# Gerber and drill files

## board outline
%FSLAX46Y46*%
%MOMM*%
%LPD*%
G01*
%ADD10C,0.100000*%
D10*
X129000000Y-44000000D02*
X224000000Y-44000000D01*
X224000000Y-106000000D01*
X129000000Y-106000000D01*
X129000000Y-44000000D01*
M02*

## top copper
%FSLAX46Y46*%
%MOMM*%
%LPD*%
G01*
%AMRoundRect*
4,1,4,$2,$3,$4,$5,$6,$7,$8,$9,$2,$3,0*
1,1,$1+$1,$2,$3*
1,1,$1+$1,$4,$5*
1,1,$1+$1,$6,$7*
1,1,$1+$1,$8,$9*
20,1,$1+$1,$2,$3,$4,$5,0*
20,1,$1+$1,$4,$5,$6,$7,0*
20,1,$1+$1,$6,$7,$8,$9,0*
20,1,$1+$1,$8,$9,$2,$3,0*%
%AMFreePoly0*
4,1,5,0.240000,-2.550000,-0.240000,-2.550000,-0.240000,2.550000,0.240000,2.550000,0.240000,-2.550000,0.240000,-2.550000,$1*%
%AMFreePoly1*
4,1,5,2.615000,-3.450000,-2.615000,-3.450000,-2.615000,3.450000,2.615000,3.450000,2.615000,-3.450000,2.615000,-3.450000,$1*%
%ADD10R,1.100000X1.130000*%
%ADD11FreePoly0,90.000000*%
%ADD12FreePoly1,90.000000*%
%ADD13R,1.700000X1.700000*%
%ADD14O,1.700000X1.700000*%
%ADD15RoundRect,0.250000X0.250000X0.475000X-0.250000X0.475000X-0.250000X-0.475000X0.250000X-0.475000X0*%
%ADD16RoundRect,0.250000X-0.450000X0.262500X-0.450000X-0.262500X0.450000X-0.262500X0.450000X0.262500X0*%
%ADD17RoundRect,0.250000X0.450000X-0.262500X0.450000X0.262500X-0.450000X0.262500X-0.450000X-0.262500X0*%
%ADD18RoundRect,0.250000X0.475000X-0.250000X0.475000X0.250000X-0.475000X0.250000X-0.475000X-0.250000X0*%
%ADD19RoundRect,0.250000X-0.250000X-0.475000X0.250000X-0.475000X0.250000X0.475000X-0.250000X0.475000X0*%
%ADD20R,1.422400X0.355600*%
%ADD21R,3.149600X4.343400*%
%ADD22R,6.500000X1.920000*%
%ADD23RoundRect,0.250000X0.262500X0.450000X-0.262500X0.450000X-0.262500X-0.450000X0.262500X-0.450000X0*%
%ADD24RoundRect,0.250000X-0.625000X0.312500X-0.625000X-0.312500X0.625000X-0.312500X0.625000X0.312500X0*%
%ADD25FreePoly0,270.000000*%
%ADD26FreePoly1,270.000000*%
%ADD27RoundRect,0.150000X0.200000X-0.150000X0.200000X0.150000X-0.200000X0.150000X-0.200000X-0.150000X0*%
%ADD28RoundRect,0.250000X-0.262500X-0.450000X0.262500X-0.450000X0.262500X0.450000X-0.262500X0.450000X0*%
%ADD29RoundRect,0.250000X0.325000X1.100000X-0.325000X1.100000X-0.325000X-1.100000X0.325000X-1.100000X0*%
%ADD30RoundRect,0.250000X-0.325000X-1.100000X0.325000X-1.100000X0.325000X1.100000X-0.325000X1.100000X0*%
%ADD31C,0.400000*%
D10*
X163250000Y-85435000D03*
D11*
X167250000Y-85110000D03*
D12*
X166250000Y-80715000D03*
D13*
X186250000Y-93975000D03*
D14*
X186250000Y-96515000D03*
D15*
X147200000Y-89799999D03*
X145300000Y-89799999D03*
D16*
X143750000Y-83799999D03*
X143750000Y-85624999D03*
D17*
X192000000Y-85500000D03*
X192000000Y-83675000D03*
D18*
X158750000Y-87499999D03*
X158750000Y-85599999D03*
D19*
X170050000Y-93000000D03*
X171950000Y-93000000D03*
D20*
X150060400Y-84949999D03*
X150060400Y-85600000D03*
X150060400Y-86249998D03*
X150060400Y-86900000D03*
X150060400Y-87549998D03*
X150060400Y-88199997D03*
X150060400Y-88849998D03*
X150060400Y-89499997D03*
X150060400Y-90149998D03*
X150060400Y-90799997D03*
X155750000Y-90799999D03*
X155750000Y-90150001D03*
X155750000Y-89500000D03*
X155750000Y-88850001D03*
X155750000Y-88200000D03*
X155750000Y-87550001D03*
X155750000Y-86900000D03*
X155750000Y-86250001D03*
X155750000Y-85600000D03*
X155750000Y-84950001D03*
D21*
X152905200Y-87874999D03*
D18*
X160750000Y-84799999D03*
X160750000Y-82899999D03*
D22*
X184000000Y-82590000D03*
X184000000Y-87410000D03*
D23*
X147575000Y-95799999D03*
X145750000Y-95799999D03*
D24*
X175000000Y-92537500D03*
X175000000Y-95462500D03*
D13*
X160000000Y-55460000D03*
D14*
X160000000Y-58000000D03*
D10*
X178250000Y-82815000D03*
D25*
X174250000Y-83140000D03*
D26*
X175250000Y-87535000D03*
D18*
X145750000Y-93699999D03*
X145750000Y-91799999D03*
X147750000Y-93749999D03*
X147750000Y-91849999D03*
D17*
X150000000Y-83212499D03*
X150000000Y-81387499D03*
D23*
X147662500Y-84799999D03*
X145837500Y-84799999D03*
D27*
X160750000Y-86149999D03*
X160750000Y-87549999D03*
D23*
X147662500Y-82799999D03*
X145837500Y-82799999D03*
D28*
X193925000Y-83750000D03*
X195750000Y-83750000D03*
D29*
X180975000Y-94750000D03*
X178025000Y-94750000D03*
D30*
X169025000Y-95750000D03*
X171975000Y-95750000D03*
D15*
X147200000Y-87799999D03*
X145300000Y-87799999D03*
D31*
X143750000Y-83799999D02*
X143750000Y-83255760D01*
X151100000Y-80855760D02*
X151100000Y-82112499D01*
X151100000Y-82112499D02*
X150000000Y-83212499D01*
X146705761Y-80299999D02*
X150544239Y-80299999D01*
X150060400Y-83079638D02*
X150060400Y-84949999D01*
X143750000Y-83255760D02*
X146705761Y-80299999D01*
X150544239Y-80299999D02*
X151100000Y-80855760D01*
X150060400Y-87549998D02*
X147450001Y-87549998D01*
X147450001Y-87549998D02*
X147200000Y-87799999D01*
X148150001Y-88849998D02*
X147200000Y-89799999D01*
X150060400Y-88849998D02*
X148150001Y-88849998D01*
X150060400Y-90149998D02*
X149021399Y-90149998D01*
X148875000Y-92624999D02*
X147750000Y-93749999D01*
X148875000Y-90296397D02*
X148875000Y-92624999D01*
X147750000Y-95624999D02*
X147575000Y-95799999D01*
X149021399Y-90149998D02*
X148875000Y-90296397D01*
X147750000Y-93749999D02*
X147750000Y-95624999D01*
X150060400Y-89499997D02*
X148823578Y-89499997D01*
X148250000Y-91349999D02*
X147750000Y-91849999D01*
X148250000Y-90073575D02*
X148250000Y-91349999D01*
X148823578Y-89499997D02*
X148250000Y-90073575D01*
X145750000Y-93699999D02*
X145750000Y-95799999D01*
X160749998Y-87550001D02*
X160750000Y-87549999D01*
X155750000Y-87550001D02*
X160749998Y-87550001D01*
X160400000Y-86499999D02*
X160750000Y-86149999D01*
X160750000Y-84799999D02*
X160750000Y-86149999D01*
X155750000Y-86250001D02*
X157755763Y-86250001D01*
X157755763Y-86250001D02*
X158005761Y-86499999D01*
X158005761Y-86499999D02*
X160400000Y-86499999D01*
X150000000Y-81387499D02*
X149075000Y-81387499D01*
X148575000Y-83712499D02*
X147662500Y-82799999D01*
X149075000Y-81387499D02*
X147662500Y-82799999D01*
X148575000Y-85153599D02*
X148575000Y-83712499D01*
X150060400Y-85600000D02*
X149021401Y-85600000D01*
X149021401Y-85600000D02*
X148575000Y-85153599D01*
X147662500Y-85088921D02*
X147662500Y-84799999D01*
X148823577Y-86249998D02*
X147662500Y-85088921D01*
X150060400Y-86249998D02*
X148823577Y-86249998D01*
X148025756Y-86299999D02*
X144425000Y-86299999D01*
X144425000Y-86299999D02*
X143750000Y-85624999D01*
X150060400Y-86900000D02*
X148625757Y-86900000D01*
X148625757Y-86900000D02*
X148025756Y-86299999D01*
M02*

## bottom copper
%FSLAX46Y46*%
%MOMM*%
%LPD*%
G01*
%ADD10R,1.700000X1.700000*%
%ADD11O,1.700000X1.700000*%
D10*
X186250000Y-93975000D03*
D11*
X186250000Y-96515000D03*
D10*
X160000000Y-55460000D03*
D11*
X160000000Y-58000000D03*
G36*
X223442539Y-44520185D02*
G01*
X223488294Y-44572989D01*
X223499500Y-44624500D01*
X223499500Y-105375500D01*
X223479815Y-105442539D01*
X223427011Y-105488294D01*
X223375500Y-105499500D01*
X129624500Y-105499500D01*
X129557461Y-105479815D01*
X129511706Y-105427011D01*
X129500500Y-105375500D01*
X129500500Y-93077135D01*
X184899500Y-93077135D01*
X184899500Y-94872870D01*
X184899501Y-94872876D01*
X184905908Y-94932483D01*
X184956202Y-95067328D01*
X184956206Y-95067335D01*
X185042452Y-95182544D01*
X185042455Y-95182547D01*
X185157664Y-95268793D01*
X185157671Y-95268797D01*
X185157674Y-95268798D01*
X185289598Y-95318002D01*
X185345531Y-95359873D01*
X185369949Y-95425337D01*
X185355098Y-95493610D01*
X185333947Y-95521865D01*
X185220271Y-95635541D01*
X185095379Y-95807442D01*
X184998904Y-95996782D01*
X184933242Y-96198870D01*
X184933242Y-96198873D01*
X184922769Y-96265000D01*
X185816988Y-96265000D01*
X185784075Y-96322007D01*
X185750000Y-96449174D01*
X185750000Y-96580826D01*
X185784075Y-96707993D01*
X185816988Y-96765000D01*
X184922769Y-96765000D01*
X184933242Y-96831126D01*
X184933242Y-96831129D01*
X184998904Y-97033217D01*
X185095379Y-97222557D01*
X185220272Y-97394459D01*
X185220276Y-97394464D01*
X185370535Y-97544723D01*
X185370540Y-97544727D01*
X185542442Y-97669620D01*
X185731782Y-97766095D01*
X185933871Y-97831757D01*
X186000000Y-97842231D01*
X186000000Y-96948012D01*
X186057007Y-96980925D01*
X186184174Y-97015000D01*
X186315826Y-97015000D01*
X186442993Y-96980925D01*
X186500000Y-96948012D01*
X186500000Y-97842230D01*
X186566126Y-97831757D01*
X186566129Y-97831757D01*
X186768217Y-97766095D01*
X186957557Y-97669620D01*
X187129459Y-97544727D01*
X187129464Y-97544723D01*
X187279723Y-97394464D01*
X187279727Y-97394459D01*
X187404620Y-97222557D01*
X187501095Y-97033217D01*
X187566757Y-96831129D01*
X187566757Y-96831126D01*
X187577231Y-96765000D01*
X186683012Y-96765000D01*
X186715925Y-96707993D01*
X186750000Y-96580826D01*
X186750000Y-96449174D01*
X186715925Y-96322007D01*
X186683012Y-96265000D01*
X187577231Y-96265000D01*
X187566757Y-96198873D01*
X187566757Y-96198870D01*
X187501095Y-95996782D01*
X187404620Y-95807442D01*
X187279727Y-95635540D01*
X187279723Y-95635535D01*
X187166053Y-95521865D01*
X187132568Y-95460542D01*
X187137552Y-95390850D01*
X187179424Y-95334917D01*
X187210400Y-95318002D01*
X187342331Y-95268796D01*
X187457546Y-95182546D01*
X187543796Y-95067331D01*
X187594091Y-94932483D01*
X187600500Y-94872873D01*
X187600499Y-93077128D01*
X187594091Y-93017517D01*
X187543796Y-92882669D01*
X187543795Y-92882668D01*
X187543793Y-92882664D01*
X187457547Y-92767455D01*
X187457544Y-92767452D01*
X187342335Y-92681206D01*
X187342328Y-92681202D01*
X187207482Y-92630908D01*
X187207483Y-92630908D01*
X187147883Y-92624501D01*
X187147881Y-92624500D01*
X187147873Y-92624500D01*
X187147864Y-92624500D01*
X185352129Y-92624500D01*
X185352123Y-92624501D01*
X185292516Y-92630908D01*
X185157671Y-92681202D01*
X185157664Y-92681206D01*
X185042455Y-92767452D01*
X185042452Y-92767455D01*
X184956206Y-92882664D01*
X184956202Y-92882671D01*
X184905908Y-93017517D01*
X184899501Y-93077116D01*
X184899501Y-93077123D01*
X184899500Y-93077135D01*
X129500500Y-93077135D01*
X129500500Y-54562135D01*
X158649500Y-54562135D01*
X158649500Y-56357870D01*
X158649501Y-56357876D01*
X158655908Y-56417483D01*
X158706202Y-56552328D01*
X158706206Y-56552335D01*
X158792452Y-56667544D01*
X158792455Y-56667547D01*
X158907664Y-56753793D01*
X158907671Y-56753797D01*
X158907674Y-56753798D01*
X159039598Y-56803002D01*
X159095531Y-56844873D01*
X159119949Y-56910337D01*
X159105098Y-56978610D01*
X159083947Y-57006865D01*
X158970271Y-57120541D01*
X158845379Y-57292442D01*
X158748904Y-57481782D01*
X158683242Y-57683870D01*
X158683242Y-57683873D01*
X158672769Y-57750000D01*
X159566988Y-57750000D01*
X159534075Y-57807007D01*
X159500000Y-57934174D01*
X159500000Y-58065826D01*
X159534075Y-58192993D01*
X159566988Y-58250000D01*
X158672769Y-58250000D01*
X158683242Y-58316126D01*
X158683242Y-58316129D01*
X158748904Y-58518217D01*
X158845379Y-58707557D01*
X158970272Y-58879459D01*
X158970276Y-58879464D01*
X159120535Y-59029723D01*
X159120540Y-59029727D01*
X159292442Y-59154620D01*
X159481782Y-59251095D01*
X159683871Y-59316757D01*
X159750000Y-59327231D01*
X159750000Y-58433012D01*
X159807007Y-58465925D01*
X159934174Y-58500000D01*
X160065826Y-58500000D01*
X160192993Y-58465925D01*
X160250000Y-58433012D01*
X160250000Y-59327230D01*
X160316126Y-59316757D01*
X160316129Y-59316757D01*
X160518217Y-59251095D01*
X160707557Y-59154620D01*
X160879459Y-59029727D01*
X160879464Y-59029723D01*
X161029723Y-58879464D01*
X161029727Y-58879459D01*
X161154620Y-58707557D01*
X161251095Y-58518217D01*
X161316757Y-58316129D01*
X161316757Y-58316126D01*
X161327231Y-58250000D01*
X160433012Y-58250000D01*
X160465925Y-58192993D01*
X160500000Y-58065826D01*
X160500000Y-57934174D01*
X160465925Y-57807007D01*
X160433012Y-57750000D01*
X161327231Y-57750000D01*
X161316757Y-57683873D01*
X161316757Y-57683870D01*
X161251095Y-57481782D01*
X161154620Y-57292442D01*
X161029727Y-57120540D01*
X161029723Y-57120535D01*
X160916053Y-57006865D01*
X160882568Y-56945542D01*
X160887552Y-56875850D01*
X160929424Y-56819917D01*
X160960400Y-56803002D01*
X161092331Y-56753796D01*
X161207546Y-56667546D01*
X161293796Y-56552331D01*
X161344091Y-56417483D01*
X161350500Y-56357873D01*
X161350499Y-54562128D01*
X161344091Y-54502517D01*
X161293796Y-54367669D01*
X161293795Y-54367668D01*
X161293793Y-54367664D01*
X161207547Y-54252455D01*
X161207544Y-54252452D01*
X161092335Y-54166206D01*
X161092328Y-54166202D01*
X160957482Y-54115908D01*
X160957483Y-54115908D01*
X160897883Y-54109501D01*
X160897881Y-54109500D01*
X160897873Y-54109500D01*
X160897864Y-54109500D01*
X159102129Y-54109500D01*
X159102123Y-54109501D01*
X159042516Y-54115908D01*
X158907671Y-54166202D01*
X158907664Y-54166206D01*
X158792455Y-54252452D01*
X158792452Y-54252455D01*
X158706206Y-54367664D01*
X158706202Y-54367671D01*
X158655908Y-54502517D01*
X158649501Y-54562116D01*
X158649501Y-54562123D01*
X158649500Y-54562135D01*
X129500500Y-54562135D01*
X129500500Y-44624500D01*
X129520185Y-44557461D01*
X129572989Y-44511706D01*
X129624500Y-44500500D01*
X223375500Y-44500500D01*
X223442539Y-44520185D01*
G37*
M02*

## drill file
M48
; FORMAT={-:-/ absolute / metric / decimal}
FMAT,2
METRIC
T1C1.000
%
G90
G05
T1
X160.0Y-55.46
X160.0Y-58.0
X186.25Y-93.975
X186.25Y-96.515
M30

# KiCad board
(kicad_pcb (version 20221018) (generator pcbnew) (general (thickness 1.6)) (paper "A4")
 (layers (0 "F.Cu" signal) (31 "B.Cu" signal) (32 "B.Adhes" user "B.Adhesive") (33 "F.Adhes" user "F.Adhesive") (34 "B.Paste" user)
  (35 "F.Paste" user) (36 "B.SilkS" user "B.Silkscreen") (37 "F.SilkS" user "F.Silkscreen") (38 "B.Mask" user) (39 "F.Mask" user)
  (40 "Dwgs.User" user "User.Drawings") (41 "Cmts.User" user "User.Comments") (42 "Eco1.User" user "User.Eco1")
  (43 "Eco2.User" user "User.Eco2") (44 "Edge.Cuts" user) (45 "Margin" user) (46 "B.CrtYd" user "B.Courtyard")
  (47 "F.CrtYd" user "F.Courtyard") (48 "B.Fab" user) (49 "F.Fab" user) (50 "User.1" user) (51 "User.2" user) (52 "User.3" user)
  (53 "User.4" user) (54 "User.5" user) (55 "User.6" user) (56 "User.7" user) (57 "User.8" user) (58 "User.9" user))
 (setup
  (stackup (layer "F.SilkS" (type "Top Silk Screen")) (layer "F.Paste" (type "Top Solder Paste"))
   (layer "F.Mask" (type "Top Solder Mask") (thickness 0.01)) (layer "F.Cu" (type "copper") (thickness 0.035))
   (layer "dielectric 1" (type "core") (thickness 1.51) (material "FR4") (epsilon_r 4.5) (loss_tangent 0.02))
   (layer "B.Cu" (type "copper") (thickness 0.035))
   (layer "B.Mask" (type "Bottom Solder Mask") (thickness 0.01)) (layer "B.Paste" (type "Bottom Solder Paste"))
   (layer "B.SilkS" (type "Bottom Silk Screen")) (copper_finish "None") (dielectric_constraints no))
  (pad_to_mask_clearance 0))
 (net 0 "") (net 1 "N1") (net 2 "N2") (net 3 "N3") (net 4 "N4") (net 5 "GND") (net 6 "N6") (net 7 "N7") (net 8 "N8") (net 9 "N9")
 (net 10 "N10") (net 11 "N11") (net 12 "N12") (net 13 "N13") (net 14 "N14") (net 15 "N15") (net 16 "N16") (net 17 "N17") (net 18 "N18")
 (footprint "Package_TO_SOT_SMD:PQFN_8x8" (layer "F.Cu") (at 166.25 81.5 90)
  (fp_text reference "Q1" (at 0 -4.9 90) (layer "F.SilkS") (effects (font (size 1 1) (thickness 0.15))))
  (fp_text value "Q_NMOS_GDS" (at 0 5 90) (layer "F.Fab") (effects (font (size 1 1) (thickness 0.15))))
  (pad "" smd rect (at -0.5 -2.25) (size 1.5 1.5) (layers "F.Paste"))
  (pad "" smd rect (at -0.5 0) (size 1.5 1.5) (layers "F.Paste"))
  (pad "" smd rect (at -0.5 2.25) (size 1.5 1.5) (layers "F.Paste"))
  (pad "" smd rect (at 2 -2.25) (size 1.5 1.5) (layers "F.Paste")) (pad "" smd rect (at 2 0) (size 1.5 1.5) (layers "F.Paste"))
  (pad "" smd rect (at 2 2.25) (size 1.5 1.5) (layers "F.Paste"))
  (pad "1" smd rect (at -3.935 -3 90) (size 1.13 1.1) (layers "F.Cu" "F.Paste" "F.Mask") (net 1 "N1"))
  (pad "2" smd custom (at -3.61 1 90) (size 0.48 5.1) (layers "F.Cu" "F.Paste" "F.Mask") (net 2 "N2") (zone_connect 2)
   (thermal_bridge_angle 45) (options (clearance outline) (anchor rect)) (primitives))
  (pad "3" smd custom (at 0.785 0 90) (size 5.23 6.9) (layers "F.Cu" "F.Mask") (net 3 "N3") (zone_connect 2) (thermal_bridge_angle 45)
   (options (clearance outline) (anchor rect)) (primitives)))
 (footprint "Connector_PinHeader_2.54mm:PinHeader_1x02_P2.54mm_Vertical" (layer "F.Cu") (at 186.25 93.975)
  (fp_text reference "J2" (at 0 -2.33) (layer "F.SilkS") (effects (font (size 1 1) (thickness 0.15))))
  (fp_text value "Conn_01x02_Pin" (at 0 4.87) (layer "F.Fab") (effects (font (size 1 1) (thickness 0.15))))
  (pad "1" thru_hole rect (at 0 0) (size 1.7 1.7) (drill 1) (layers "*.Cu" "*.Mask") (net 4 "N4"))
  (pad "2" thru_hole oval (at 0 2.54) (size 1.7 1.7) (drill 1) (layers "*.Cu" "*.Mask") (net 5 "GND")))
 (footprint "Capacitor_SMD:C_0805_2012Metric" (layer "F.Cu") (at 146.25 89.799999 180)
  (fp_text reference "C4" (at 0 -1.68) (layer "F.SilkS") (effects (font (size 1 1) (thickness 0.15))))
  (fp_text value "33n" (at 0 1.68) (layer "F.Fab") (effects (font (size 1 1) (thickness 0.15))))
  (pad "1" smd roundrect (at -0.95 0 180) (size 1 1.45) (layers "F.Cu" "F.Paste" "F.Mask") (roundrect_rratio 0.25) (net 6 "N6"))
  (pad "2" smd roundrect (at 0.95 0 180) (size 1 1.45) (layers "F.Cu" "F.Paste" "F.Mask") (roundrect_rratio 0.25) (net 5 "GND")))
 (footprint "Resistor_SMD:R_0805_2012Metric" (layer "F.Cu") (at 143.75 84.712499 -90)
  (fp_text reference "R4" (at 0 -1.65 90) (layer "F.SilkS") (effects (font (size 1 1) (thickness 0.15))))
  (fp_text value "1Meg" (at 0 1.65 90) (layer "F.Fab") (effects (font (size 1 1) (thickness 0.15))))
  (pad "1" smd roundrect (at -0.9125 0 270) (size 1.025 1.4) (layers "F.Cu" "F.Paste" "F.Mask") (roundrect_rratio 0.243902) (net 2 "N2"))
  (pad "2" smd roundrect (at 0.9125 0 270) (size 1.025 1.4) (layers "F.Cu" "F.Paste" "F.Mask") (roundrect_rratio 0.243902) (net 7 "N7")))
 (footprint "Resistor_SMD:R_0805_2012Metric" (layer "F.Cu") (at 192 84.5875 90)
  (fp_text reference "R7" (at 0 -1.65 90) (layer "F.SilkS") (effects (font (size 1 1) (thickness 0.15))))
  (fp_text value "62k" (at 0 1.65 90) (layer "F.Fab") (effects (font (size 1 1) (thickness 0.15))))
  (pad "1" smd roundrect (at -0.9125 0 90) (size 1.025 1.4) (layers "F.Cu" "F.Paste" "F.Mask") (roundrect_rratio 0.243902) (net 4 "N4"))
  (pad "2" smd roundrect (at 0.9125 0 90) (size 1.025 1.4) (layers "F.Cu" "F.Paste" "F.Mask") (roundrect_rratio 0.243902) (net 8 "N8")))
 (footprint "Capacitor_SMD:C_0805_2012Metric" (layer "F.Cu") (at 158.75 86.549999 90)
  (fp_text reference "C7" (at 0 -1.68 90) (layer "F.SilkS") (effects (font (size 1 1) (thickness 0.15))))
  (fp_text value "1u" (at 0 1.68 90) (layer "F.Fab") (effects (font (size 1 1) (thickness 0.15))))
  (pad "1" smd roundrect (at -0.95 0 90) (size 1 1.45) (layers "F.Cu" "F.Paste" "F.Mask") (roundrect_rratio 0.25) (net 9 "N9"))
  (pad "2" smd roundrect (at 0.95 0 90) (size 1 1.45) (layers "F.Cu" "F.Paste" "F.Mask") (roundrect_rratio 0.25) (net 5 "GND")))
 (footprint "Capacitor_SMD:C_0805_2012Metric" (layer "F.Cu") (at 171 93)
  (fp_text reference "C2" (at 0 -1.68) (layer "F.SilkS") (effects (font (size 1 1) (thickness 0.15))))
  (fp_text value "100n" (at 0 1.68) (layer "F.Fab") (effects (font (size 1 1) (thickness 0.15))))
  (pad "1" smd roundrect (at -0.95 0) (size 1 1.45) (layers "F.Cu" "F.Paste" "F.Mask") (roundrect_rratio 0.25) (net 2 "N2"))
  (pad "2" smd roundrect (at 0.95 0) (size 1 1.45) (layers "F.Cu" "F.Paste" "F.Mask") (roundrect_rratio 0.25) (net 5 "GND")))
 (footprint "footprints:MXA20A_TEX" (layer "F.Cu") (at 152.9052 87.874999)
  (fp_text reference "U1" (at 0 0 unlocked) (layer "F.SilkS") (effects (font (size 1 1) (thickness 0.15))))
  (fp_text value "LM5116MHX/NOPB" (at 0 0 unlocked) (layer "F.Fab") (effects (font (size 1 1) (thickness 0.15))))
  (pad "1" smd rect (at -2.8448 -2.925) (size 1.4224 0.3556) (layers "F.Cu" "F.Paste" "F.Mask") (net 2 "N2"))
  (pad "2" smd rect (at -2.8448 -2.274999) (size 1.4224 0.3556) (layers "F.Cu" "F.Paste" "F.Mask") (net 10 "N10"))
  (pad "3" smd rect (at -2.8448 -1.625001) (size 1.4224 0.3556) (layers "F.Cu" "F.Paste" "F.Mask") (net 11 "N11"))
  (pad "4" smd rect (at -2.8448 -0.974999) (size 1.4224 0.3556) (layers "F.Cu" "F.Paste" "F.Mask") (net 7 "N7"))
  (pad "5" smd rect (at -2.8448 -0.325001) (size 1.4224 0.3556) (layers "F.Cu" "F.Paste" "F.Mask") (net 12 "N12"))
  (pad "6" smd rect (at -2.8448 0.324998) (size 1.4224 0.3556) (layers "F.Cu" "F.Paste" "F.Mask") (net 5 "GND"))
  (pad "7" smd rect (at -2.8448 0.974999) (size 1.4224 0.3556) (layers "F.Cu" "F.Paste" "F.Mask") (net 6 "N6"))
  (pad "8" smd rect (at -2.8448 1.624998) (size 1.4224 0.3556) (layers "F.Cu" "F.Paste" "F.Mask") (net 8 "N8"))
  (pad "9" smd rect (at -2.8448 2.274999) (size 1.4224 0.3556) (layers "F.Cu" "F.Paste" "F.Mask") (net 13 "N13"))
  (pad "10" smd rect (at -2.8448 2.924998) (size 1.4224 0.3556) (layers "F.Cu" "F.Paste" "F.Mask") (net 4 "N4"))
  (pad "11" smd rect (at 2.8448 2.925) (size 1.4224 0.3556) (layers "F.Cu" "F.Paste" "F.Mask") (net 5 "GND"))
  (pad "12" smd rect (at 2.8448 2.275002) (size 1.4224 0.3556) (layers "F.Cu" "F.Paste" "F.Mask") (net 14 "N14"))
  (pad "13" smd rect (at 2.8448 1.625001) (size 1.4224 0.3556) (layers "F.Cu" "F.Paste" "F.Mask") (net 5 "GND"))
  (pad "14" smd rect (at 2.8448 0.975002) (size 1.4224 0.3556) (layers "F.Cu" "F.Paste" "F.Mask") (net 5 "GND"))
  (pad "15" smd rect (at 2.8448 0.325001) (size 1.4224 0.3556) (layers "F.Cu" "F.Paste" "F.Mask") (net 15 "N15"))
  (pad "16" smd rect (at 2.8448 -0.324998) (size 1.4224 0.3556) (layers "F.Cu" "F.Paste" "F.Mask") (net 9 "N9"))
  (pad "17" smd rect (at 2.8448 -0.974999) (size 1.4224 0.3556) (layers "F.Cu" "F.Paste" "F.Mask") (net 5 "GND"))
  (pad "18" smd rect (at 2.8448 -1.624998) (size 1.4224 0.3556) (layers "F.Cu" "F.Paste" "F.Mask") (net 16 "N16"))
  (pad "19" smd rect (at 2.8448 -2.274999) (size 1.4224 0.3556) (layers "F.Cu" "F.Paste" "F.Mask") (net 1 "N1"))
  (pad "20" smd rect (at 2.8448 -2.924998) (size 1.4224 0.3556) (layers "F.Cu" "F.Paste" "F.Mask") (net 3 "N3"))
  (pad "21" smd rect (at 0 0) (size 3.1496 4.3434) (layers "F.Cu" "F.Paste" "F.Mask") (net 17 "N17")))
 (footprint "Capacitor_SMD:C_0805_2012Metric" (layer "F.Cu") (at 160.75 83.849999 90)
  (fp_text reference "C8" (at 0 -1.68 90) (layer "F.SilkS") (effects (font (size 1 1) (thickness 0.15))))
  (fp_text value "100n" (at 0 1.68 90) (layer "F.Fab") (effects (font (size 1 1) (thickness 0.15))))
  (pad "1" smd roundrect (at -0.95 0 90) (size 1 1.45) (layers "F.Cu" "F.Paste" "F.Mask") (roundrect_rratio 0.25) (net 16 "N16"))
  (pad "2" smd roundrect (at 0.95 0 90) (size 1 1.45) (layers "F.Cu" "F.Paste" "F.Mask") (roundrect_rratio 0.25) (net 3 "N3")))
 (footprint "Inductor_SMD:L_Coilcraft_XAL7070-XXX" (layer "F.Cu") (at 184 85 -90)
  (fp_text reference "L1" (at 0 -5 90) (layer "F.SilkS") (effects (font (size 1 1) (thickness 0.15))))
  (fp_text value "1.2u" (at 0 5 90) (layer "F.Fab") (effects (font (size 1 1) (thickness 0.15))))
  (pad "1" smd rect (at -2.41 0 270) (size 1.92 6.5) (layers "F.Cu" "F.Paste" "F.Mask") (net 3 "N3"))
  (pad "2" smd rect (at 2.41 0 270) (size 1.92 6.5) (layers "F.Cu" "F.Paste" "F.Mask") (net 4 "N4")))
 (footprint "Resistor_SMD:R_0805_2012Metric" (layer "F.Cu") (at 146.6625 95.799999 180)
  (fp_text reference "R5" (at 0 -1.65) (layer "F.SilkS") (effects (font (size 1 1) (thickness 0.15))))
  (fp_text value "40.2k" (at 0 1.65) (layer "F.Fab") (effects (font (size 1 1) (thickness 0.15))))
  (pad "1" smd roundrect (at -0.9125 0 180) (size 1.025 1.4) (layers "F.Cu" "F.Paste" "F.Mask") (roundrect_rratio 0.243902) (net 13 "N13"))
  (pad "2" smd roundrect (at 0.9125 0 180) (size 1.025 1.4) (layers "F.Cu" "F.Paste" "F.Mask") (roundrect_rratio 0.243902) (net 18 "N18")))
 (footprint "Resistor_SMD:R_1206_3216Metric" (layer "F.Cu") (at 175 94 -90)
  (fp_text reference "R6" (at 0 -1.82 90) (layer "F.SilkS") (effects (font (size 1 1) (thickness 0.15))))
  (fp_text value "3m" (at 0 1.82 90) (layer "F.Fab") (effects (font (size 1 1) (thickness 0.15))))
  (pad "1" smd roundrect (at -1.4625 0 270) (size 1.125 1.75) (layers "F.Cu" "F.Paste" "F.Mask") (roundrect_rratio 0.222222) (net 14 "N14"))
  (pad "2" smd roundrect (at 1.4625 0 270) (size 1.125 1.75) (layers "F.Cu" "F.Paste" "F.Mask") (roundrect_rratio 0.222222) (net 5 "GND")))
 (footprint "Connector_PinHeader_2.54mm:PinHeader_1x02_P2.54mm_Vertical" (layer "F.Cu") (at 160 55.46)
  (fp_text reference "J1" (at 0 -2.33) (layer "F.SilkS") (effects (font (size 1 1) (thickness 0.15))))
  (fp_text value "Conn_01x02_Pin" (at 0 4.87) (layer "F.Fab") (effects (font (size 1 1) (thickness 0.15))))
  (pad "1" thru_hole rect (at 0 0) (size 1.7 1.7) (drill 1) (layers "*.Cu" "*.Mask") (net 2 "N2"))
  (pad "2" thru_hole oval (at 0 2.54) (size 1.7 1.7) (drill 1) (layers "*.Cu" "*.Mask") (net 5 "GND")))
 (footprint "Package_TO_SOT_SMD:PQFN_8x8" (layer "F.Cu") (at 175.25 86.75 -90)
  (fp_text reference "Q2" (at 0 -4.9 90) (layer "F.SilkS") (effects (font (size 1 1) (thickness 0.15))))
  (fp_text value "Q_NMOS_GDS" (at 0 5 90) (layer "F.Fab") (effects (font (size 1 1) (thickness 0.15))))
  (pad "" smd rect (at -0.5 -2.25 180) (size 1.5 1.5) (layers "F.Paste"))
  (pad "" smd rect (at -0.5 0 180) (size 1.5 1.5) (layers "F.Paste"))
  (pad "" smd rect (at -0.5 2.25 180) (size 1.5 1.5) (layers "F.Paste"))
  (pad "" smd rect (at 2 -2.25 180) (size 1.5 1.5) (layers "F.Paste"))
  (pad "" smd rect (at 2 0 180) (size 1.5 1.5) (layers "F.Paste"))
  (pad "" smd rect (at 2 2.25 180) (size 1.5 1.5) (layers "F.Paste"))
  (pad "1" smd rect (at -3.935 -3 270) (size 1.13 1.1) (layers "F.Cu" "F.Paste" "F.Mask") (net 15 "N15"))
  (pad "2" smd custom (at -3.61 1 270) (size 0.48 5.1) (layers "F.Cu" "F.Paste" "F.Mask") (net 3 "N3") (zone_connect 2)
   (thermal_bridge_angle 45) (options (clearance outline) (anchor rect)) (primitives))
  (pad "3" smd custom (at 0.785 0 270) (size 5.23 6.9) (layers "F.Cu" "F.Mask") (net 14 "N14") (zone_connect 2) (thermal_bridge_angle 45)
   (options (clearance outline) (anchor rect)) (primitives)))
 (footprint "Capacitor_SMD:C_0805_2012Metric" (layer "F.Cu") (at 145.75 92.749999 90)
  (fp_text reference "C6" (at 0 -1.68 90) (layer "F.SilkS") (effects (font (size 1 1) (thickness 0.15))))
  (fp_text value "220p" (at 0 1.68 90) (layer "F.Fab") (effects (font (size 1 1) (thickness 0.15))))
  (pad "1" smd roundrect (at -0.95 0 90) (size 1 1.45) (layers "F.Cu" "F.Paste" "F.Mask") (roundrect_rratio 0.25) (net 18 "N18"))
  (pad "2" smd roundrect (at 0.95 0 90) (size 1 1.45) (layers "F.Cu" "F.Paste" "F.Mask") (roundrect_rratio 0.25) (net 8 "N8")))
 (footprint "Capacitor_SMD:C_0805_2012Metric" (layer "F.Cu") (at 147.75 92.799999 90)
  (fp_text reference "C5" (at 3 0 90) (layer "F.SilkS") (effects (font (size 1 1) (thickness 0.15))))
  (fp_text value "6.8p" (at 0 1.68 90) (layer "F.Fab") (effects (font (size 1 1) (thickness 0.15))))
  (pad "1" smd roundrect (at -0.95 0 90) (size 1 1.45) (layers "F.Cu" "F.Paste" "F.Mask") (roundrect_rratio 0.25) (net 13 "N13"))
  (pad "2" smd roundrect (at 0.95 0 90) (size 1 1.45) (layers "F.Cu" "F.Paste" "F.Mask") (roundrect_rratio 0.25) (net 8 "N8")))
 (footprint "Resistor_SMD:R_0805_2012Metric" (layer "F.Cu") (at 150 82.299999 90)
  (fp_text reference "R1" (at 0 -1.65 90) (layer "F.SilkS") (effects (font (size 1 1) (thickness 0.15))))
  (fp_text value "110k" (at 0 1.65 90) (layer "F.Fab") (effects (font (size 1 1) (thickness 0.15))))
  (pad "1" smd roundrect (at -0.9125 0 90) (size 1.025 1.4) (layers "F.Cu" "F.Paste" "F.Mask") (roundrect_rratio 0.243902) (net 2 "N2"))
  (pad "2" smd roundrect (at 0.9125 0 90) (size 1.025 1.4) (layers "F.Cu" "F.Paste" "F.Mask") (roundrect_rratio 0.243902) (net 10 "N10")))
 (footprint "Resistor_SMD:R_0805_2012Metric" (layer "F.Cu") (at 146.75 84.799999 180)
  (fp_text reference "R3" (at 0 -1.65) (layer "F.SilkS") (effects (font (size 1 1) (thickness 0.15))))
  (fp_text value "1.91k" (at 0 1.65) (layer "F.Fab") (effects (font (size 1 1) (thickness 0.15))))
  (pad "1" smd roundrect (at -0.9125 0 180) (size 1.025 1.4) (layers "F.Cu" "F.Paste" "F.Mask") (roundrect_rratio 0.243902) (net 11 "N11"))
  (pad "2" smd roundrect (at 0.9125 0 180) (size 1.025 1.4) (layers "F.Cu" "F.Paste" "F.Mask") (roundrect_rratio 0.243902) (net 5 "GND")))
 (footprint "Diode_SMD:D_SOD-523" (layer "F.Cu") (at 160.75 86.849999 -90)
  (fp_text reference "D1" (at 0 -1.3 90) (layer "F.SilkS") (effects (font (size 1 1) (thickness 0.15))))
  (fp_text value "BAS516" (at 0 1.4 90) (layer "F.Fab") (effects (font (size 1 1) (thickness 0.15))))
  (pad "1" smd roundrect (at -0.7 0 90) (size 0.6 0.7) (layers "F.Cu" "F.Paste" "F.Mask") (roundrect_rratio 0.25) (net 16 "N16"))
  (pad "2" smd roundrect (at 0.7 0 90) (size 0.6 0.7) (layers "F.Cu" "F.Paste" "F.Mask") (roundrect_rratio 0.25) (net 9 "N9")))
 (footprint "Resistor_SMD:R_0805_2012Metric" (layer "F.Cu") (at 146.75 82.799999 180)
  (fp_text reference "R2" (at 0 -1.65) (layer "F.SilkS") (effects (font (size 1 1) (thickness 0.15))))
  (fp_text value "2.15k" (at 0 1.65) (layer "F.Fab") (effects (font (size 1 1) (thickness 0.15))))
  (pad "1" smd roundrect (at -0.9125 0 180) (size 1.025 1.4) (layers "F.Cu" "F.Paste" "F.Mask") (roundrect_rratio 0.243902) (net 10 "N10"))
  (pad "2" smd roundrect (at 0.9125 0 180) (size 1.025 1.4) (layers "F.Cu" "F.Paste" "F.Mask") (roundrect_rratio 0.243902) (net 5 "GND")))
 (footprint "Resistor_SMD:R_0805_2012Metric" (layer "F.Cu") (at 194.8375 83.75)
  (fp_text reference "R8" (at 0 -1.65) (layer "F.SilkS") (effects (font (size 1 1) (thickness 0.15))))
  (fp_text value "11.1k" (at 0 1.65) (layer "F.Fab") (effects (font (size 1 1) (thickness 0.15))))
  (pad "1" smd roundrect (at -0.9125 0) (size 1.025 1.4) (layers "F.Cu" "F.Paste" "F.Mask") (roundrect_rratio 0.243902) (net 8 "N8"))
  (pad "2" smd roundrect (at 0.9125 0) (size 1.025 1.4) (layers "F.Cu" "F.Paste" "F.Mask") (roundrect_rratio 0.243902) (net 5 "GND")))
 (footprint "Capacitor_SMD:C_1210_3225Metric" (layer "F.Cu") (at 179.5 94.75 180)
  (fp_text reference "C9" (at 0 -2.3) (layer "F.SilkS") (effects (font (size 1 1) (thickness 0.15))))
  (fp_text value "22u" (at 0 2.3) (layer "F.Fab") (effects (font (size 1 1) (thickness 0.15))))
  (pad "1" smd roundrect (at -1.475 0 180) (size 1.15 2.7) (layers "F.Cu" "F.Paste" "F.Mask") (roundrect_rratio 0.217391) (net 4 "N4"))
  (pad "2" smd roundrect (at 1.475 0 180) (size 1.15 2.7) (layers "F.Cu" "F.Paste" "F.Mask") (roundrect_rratio 0.217391) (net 5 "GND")))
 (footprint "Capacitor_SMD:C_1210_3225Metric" (layer "F.Cu") (at 170.5 95.75)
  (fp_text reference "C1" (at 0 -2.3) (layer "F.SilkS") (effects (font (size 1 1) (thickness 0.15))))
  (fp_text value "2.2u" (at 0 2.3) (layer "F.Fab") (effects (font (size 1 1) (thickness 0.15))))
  (pad "1" smd roundrect (at -1.475 0) (size 1.15 2.7) (layers "F.Cu" "F.Paste" "F.Mask") (roundrect_rratio 0.217391) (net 2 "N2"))
  (pad "2" smd roundrect (at 1.475 0) (size 1.15 2.7) (layers "F.Cu" "F.Paste" "F.Mask") (roundrect_rratio 0.217391) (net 5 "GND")))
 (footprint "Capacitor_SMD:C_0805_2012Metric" (layer "F.Cu") (at 146.25 87.799999 180)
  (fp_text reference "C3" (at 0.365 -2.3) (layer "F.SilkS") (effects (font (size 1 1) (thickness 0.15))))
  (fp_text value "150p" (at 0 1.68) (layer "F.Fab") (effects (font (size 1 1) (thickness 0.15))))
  (pad "1" smd roundrect (at -0.95 0 180) (size 1 1.45) (layers "F.Cu" "F.Paste" "F.Mask") (roundrect_rratio 0.25) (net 12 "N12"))
  (pad "2" smd roundrect (at 0.95 0 180) (size 1 1.45) (layers "F.Cu" "F.Paste" "F.Mask") (roundrect_rratio 0.25) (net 5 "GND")))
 (gr_rect (start 129 44) (end 224 106) (stroke (width 0.1) (type default)) (fill none) (layer "Edge.Cuts"))
 (segment (start 143.75 83.799999) (end 143.75 83.25576) (width 0.4) (layer "F.Cu") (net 2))
 (segment (start 151.1 80.85576) (end 151.1 82.112499) (width 0.4) (layer "F.Cu") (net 2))
 (segment (start 151.1 82.112499) (end 150 83.212499) (width 0.4) (layer "F.Cu") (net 2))
 (segment (start 146.705761 80.299999) (end 150.544239 80.299999) (width 0.4) (layer "F.Cu") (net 2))
 (segment (start 150.0604 83.079638) (end 150.0604 84.949999) (width 0.4) (layer "F.Cu") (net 2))
 (segment (start 143.75 83.25576) (end 146.705761 80.299999) (width 0.4) (layer "F.Cu") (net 2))
 (segment (start 150.544239 80.299999) (end 151.1 80.85576) (width 0.4) (layer "F.Cu") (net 2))
 (segment (start 150.0604 87.549998) (end 147.450001 87.549998) (width 0.4) (layer "F.Cu") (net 12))
 (segment (start 147.450001 87.549998) (end 147.2 87.799999) (width 0.4) (layer "F.Cu") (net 12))
 (segment (start 148.150001 88.849998) (end 147.2 89.799999) (width 0.4) (layer "F.Cu") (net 6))
 (segment (start 150.0604 88.849998) (end 148.150001 88.849998) (width 0.4) (layer "F.Cu") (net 6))
 (segment (start 150.0604 90.149998) (end 149.021399 90.149998) (width 0.4) (layer "F.Cu") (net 13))
 (segment (start 148.875 92.624999) (end 147.75 93.749999) (width 0.4) (layer "F.Cu") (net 13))
 (segment (start 148.875 90.296397) (end 148.875 92.624999) (width 0.4) (layer "F.Cu") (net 13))
 (segment (start 147.75 95.624999) (end 147.575 95.799999) (width 0.4) (layer "F.Cu") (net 13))
 (segment (start 149.021399 90.149998) (end 148.875 90.296397) (width 0.4) (layer "F.Cu") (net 13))
 (segment (start 147.75 93.749999) (end 147.75 95.624999) (width 0.4) (layer "F.Cu") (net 13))
 (segment (start 150.0604 89.499997) (end 148.823578 89.499997) (width 0.4) (layer "F.Cu") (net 8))
 (segment (start 148.25 91.349999) (end 147.75 91.849999) (width 0.4) (layer "F.Cu") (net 8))
 (segment (start 148.25 90.073575) (end 148.25 91.349999) (width 0.4) (layer "F.Cu") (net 8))
 (segment (start 148.823578 89.499997) (end 148.25 90.073575) (width 0.4) (layer "F.Cu") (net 8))
 (segment (start 145.75 93.699999) (end 145.75 95.799999) (width 0.4) (layer "F.Cu") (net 18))
 (segment (start 160.749998 87.550001) (end 160.75 87.549999) (width 0.4) (layer "F.Cu") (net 9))
 (segment (start 155.75 87.550001) (end 160.749998 87.550001) (width 0.4) (layer "F.Cu") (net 9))
 (segment (start 160.4 86.499999) (end 160.75 86.149999) (width 0.4) (layer "F.Cu") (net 16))
 (segment (start 160.75 84.799999) (end 160.75 86.149999) (width 0.4) (layer "F.Cu") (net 16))
 (segment (start 155.75 86.250001) (end 157.755763 86.250001) (width 0.4) (layer "F.Cu") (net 16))
 (segment (start 157.755763 86.250001) (end 158.005761 86.499999) (width 0.4) (layer "F.Cu") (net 16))
 (segment (start 158.005761 86.499999) (end 160.4 86.499999) (width 0.4) (layer "F.Cu") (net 16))
 (segment (start 150 81.387499) (end 149.075 81.387499) (width 0.4) (layer "F.Cu") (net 10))
 (segment (start 148.575 83.712499) (end 147.6625 82.799999) (width 0.4) (layer "F.Cu") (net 10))
 (segment (start 149.075 81.387499) (end 147.6625 82.799999) (width 0.4) (layer "F.Cu") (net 10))
 (segment (start 148.575 85.153599) (end 148.575 83.712499) (width 0.4) (layer "F.Cu") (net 10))
 (segment (start 150.0604 85.6) (end 149.021401 85.6) (width 0.4) (layer "F.Cu") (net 10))
 (segment (start 149.021401 85.6) (end 148.575 85.153599) (width 0.4) (layer "F.Cu") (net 10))
 (segment (start 147.6625 85.088921) (end 147.6625 84.799999) (width 0.4) (layer "F.Cu") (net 11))
 (segment (start 148.823577 86.249998) (end 147.6625 85.088921) (width 0.4) (layer "F.Cu") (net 11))
 (segment (start 150.0604 86.249998) (end 148.823577 86.249998) (width 0.4) (layer "F.Cu") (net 11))
 (segment (start 148.025756 86.299999) (end 144.425 86.299999) (width 0.4) (layer "F.Cu") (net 7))
 (segment (start 144.425 86.299999) (end 143.75 85.624999) (width 0.4) (layer "F.Cu") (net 7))
 (segment (start 150.0604 86.9) (end 148.625757 86.9) (width 0.4) (layer "F.Cu") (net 7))
 (segment (start 148.625757 86.9) (end 148.025756 86.299999) (width 0.4) (layer "F.Cu") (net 7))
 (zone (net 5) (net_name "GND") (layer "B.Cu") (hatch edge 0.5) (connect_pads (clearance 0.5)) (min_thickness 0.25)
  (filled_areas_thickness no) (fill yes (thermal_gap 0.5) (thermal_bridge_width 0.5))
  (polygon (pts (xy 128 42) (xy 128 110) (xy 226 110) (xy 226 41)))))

